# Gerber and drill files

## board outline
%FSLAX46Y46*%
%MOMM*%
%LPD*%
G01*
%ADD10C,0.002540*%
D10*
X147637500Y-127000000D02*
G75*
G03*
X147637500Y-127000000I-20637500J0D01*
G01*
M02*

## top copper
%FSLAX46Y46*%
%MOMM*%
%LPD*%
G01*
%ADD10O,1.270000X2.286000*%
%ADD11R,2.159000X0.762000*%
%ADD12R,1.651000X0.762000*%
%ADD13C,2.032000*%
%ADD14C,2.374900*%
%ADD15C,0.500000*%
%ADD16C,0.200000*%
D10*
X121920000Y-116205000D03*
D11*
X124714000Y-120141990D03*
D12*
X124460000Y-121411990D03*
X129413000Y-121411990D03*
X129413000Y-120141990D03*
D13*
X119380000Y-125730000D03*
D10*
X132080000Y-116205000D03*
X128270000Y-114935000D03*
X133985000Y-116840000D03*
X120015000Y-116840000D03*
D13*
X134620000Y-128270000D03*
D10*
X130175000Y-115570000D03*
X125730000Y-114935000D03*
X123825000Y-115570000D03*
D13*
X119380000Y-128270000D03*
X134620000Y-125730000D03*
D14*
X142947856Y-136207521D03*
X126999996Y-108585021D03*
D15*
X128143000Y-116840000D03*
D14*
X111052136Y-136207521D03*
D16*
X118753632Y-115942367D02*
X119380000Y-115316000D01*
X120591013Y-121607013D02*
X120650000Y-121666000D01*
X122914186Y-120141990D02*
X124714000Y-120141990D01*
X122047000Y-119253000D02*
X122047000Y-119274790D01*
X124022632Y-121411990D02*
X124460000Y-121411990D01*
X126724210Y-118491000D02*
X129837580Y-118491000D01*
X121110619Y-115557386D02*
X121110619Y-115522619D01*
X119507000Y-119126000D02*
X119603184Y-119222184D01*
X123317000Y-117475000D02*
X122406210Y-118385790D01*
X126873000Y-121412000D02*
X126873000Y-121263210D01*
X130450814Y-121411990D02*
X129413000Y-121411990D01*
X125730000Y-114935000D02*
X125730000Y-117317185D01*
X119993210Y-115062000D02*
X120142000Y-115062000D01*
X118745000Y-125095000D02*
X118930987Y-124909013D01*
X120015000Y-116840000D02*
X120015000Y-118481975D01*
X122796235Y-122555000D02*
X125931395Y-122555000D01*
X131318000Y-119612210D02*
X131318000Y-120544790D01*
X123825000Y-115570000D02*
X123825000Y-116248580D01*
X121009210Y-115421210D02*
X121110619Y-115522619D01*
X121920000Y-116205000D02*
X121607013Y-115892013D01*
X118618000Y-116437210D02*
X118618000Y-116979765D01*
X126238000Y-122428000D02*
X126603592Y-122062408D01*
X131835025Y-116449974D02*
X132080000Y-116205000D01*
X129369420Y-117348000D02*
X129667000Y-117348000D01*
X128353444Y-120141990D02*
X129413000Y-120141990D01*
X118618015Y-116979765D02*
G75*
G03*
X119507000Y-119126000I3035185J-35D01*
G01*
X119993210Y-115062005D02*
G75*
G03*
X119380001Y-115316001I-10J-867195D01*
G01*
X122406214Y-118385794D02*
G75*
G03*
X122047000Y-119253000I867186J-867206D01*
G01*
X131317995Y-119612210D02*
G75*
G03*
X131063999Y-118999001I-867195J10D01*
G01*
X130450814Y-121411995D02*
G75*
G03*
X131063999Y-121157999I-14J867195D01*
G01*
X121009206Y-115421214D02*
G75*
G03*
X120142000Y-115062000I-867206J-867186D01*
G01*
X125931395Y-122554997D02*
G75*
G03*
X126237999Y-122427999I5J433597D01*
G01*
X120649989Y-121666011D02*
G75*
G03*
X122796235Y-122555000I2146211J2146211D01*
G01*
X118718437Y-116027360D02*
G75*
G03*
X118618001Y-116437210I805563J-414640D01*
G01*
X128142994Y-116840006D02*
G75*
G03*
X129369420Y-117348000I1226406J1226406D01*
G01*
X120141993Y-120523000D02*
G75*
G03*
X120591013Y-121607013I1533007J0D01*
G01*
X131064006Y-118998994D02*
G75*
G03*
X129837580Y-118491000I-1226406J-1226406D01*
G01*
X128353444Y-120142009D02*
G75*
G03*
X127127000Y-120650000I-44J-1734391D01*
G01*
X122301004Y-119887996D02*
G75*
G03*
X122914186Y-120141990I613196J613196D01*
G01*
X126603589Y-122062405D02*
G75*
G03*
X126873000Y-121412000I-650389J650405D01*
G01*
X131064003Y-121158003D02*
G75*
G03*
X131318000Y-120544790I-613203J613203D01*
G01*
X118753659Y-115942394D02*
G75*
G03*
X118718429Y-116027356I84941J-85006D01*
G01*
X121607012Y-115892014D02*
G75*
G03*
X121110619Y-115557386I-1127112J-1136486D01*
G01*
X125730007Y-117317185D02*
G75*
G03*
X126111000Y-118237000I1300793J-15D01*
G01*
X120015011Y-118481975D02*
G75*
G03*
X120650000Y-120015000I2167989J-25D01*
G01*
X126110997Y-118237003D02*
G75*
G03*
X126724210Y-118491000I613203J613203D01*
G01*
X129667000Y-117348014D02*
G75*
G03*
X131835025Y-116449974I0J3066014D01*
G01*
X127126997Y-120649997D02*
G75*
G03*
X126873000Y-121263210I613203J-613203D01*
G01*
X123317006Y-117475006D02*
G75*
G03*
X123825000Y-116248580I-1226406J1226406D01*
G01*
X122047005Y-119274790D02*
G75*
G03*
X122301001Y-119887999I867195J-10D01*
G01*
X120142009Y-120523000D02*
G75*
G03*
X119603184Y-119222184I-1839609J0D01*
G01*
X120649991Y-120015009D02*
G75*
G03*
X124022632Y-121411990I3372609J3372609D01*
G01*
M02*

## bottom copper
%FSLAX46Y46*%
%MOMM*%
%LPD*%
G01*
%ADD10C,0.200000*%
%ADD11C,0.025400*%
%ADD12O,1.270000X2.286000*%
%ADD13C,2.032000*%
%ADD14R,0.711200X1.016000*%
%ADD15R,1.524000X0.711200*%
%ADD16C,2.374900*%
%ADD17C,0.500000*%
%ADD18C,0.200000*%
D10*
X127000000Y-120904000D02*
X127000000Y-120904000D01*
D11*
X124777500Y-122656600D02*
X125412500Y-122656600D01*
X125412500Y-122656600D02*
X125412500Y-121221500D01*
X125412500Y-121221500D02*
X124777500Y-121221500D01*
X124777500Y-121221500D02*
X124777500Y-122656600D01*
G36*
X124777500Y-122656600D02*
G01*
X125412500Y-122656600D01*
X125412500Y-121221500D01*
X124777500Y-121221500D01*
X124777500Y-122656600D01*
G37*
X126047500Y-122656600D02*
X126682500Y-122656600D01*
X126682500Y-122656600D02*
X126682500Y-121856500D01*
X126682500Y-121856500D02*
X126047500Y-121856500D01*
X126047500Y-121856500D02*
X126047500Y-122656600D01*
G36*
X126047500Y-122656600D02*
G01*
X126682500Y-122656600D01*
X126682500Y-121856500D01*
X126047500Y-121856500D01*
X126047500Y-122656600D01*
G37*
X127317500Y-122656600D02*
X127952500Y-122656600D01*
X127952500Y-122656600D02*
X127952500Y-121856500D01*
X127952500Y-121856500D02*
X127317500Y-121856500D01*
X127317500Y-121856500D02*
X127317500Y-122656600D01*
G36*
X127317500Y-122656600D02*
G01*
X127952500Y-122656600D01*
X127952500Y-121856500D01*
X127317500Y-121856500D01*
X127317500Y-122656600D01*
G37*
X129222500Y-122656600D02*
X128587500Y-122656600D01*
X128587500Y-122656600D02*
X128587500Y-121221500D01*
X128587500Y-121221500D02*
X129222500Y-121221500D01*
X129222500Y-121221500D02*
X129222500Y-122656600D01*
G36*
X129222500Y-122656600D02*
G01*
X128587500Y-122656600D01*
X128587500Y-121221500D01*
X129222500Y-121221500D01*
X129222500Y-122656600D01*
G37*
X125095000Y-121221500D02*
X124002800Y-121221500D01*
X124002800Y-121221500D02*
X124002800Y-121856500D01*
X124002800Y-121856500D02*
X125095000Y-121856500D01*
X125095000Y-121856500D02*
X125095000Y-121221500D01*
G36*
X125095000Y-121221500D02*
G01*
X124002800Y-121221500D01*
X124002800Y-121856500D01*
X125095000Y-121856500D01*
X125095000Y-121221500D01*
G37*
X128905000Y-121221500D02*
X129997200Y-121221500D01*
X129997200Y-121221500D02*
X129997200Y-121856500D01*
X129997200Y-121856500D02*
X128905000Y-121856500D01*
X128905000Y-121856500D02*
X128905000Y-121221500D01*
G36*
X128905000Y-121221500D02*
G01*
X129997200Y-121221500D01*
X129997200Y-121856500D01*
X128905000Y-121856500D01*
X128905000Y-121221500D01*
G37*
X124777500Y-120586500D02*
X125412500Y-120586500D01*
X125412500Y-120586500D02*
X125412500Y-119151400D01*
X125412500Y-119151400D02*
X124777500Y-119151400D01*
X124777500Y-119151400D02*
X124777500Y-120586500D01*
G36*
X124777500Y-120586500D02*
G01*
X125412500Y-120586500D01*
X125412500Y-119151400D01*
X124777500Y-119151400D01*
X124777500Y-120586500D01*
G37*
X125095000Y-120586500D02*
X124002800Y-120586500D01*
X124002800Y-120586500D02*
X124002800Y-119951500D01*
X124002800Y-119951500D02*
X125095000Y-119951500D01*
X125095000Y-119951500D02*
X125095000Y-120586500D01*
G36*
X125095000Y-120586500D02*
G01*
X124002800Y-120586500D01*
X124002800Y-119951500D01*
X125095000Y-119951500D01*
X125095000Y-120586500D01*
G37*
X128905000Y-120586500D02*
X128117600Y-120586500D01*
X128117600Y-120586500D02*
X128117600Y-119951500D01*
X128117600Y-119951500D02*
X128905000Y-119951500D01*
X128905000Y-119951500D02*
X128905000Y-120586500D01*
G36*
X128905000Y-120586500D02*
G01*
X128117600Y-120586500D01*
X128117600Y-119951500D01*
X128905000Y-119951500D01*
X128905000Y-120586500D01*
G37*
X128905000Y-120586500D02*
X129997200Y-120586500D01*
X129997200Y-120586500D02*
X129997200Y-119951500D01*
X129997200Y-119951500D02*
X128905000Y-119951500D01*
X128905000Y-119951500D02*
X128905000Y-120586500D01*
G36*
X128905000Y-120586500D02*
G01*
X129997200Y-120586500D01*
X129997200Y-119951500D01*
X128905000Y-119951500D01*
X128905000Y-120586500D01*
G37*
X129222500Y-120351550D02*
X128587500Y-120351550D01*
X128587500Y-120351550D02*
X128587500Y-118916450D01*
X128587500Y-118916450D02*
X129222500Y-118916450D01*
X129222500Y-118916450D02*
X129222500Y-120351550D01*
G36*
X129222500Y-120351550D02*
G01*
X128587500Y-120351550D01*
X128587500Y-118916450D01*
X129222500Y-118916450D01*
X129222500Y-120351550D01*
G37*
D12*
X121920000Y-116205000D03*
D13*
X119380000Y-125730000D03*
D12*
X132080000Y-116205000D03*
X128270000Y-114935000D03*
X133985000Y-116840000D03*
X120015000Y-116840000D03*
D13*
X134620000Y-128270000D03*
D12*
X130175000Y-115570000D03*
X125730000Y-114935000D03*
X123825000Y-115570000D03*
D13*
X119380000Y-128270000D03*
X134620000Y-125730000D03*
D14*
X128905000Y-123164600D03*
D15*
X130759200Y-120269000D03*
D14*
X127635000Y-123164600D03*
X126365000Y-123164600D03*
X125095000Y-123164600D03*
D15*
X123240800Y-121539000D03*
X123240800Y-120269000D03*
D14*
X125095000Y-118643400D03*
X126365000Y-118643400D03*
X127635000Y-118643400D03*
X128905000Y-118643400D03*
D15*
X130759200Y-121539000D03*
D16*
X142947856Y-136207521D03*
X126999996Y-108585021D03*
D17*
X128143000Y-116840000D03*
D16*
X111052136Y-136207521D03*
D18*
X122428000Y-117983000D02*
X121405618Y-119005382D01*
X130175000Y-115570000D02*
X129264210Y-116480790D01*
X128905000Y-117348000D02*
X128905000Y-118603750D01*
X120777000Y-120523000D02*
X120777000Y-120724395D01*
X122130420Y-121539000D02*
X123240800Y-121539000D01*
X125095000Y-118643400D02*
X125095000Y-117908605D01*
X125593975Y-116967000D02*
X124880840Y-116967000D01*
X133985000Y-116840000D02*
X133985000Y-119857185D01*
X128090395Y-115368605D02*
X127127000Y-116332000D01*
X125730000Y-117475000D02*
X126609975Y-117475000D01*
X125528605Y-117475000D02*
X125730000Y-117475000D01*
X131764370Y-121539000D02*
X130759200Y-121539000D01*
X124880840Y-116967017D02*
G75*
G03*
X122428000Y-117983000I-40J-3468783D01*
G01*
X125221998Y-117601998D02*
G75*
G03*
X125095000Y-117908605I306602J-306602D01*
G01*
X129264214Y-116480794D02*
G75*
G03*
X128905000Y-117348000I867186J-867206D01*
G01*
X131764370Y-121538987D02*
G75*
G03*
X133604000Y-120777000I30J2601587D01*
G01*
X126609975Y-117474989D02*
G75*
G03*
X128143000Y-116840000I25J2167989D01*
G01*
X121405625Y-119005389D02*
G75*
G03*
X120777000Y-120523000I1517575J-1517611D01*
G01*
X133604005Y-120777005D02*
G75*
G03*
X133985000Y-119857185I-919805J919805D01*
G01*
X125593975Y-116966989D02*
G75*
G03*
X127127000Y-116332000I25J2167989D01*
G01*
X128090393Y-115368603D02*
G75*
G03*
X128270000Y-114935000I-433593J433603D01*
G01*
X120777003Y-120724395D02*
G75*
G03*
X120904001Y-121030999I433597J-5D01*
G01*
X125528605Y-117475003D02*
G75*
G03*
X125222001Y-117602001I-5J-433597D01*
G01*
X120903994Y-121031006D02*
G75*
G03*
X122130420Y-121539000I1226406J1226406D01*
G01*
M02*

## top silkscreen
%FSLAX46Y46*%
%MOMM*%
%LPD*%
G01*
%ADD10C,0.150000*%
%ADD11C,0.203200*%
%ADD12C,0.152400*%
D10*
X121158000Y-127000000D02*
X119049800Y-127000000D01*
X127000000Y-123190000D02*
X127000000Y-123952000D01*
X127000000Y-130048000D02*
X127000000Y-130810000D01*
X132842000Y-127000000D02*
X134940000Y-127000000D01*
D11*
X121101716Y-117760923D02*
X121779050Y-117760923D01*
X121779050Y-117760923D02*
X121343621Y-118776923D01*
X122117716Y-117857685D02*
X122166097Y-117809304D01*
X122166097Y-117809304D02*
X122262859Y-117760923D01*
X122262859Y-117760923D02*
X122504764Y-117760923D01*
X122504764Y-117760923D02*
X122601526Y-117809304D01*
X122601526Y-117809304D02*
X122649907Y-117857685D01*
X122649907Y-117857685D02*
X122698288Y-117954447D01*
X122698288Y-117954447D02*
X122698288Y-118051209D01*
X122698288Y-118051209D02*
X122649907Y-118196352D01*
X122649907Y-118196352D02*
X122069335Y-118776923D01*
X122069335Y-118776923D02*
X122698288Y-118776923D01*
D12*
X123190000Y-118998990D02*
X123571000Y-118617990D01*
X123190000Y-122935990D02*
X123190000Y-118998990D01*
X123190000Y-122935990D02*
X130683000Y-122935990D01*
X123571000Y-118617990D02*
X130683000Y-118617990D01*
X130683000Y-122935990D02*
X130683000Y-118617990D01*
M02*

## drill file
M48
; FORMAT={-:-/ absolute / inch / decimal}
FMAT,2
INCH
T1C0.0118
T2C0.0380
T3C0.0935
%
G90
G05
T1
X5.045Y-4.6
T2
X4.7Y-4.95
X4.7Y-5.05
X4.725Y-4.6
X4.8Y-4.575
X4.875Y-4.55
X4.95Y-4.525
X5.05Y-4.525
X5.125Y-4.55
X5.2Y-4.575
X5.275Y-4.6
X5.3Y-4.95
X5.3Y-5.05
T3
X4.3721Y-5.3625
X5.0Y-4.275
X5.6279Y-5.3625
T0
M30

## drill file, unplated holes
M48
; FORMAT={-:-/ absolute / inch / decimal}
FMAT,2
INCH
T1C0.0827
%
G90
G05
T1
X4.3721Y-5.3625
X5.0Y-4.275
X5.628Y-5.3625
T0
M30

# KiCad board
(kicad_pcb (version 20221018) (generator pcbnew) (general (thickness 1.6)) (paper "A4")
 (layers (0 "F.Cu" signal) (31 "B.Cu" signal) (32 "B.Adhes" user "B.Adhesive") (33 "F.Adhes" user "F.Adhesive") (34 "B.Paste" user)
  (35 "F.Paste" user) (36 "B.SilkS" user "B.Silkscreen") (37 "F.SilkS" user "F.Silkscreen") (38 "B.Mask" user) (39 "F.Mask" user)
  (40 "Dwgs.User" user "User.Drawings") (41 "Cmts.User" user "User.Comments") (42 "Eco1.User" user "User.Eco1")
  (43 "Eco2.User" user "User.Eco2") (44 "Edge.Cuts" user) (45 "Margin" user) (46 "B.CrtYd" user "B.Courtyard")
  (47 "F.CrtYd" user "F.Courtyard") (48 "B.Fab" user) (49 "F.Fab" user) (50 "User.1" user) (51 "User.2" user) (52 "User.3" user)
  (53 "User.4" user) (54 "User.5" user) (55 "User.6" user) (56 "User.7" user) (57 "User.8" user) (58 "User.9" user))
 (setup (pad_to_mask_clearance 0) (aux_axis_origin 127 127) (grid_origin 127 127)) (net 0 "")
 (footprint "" (layer "F.Cu") (at 121.92 116.205)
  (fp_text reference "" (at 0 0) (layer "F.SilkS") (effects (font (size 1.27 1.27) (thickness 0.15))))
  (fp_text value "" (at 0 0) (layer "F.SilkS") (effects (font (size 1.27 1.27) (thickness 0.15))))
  (pad "1" thru_hole oval (at 0 0) (size 1.27 2.286) (drill 0.9652) (layers "*.Cu" "*.Mask") (thermal_bridge_angle 45)))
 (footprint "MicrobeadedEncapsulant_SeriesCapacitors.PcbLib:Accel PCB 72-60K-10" (layer "F.Cu") (at 127 120.904)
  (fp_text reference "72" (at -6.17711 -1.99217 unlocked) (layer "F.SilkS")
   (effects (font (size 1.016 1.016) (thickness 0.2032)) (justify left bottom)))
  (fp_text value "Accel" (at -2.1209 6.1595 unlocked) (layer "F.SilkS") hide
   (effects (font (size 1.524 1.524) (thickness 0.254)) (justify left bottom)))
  (fp_line (start -3.81 -1.90501) (end -3.429 -2.28601) (stroke (width 0.1524) (type solid)) (layer "F.SilkS"))
  (fp_line (start -3.81 2.03199) (end -3.81 -1.90501) (stroke (width 0.1524) (type solid)) (layer "F.SilkS"))
  (fp_line (start -3.81 2.03199) (end 3.683 2.03199) (stroke (width 0.1524) (type solid)) (layer "F.SilkS"))
  (fp_line (start -3.429 -2.28601) (end 3.683 -2.28601) (stroke (width 0.1524) (type solid)) (layer "F.SilkS"))
  (fp_line (start 3.683 2.03199) (end 3.683 -2.28601) (stroke (width 0.1524) (type solid)) (layer "F.SilkS"))
  (pad "1" smd rect (at -2.286 -0.76201 90) (size 0.762 2.159) (layers "F.Cu" "F.Paste" "F.Mask") (solder_mask_margin 0.1016)
   (thermal_bridge_angle 45))
  (pad "2" smd rect (at -2.54 0.50799 90) (size 0.762 1.651) (layers "F.Cu" "F.Paste" "F.Mask") (solder_mask_margin 0.1016)
   (thermal_bridge_angle 45))
  (pad "3" smd rect (at 2.413 0.50799 90) (size 0.762 1.651) (layers "F.Cu" "F.Paste" "F.Mask") (solder_mask_margin 0.1016)
   (thermal_bridge_angle 45))
  (pad "4" smd rect (at 2.413 -0.76201 90) (size 0.762 1.651) (layers "F.Cu" "F.Paste" "F.Mask") (solder_mask_margin 0.1016)
   (thermal_bridge_angle 45)))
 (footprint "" (layer "F.Cu") (at 119.38 125.73)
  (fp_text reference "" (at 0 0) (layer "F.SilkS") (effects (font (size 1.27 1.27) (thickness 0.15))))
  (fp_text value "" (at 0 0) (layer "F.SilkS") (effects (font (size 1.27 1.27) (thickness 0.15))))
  (pad "1" thru_hole circle (at 0 0) (size 2.032 2.032) (drill 0.9652) (layers "*.Cu" "*.Mask")))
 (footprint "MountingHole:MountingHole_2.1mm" (layer "F.Cu") (at 142.9512 136.2075)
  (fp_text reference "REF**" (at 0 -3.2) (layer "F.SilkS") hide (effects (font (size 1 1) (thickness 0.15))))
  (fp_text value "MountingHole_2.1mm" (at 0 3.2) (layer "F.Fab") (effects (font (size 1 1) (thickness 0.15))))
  (pad "" np_thru_hole circle (at 0 0) (size 2.1 2.1) (drill 2.1) (layers "*.Cu" "*.Mask")))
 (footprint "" (layer "F.Cu") (at 132.08 116.205)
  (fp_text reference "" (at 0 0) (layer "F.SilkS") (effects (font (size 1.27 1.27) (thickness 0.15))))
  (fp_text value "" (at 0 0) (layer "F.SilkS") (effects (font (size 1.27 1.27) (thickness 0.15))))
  (pad "1" thru_hole oval (at 0 0) (size 1.27 2.286) (drill 0.9652) (layers "*.Cu" "*.Mask") (thermal_bridge_angle 45)))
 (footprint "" (layer "F.Cu") (at 128.27 114.935)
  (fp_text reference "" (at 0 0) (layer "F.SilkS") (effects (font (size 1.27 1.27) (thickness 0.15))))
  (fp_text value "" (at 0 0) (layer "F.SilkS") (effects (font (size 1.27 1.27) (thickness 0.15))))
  (pad "1" thru_hole oval (at 0 0) (size 1.27 2.286) (drill 0.9652) (layers "*.Cu" "*.Mask") (thermal_bridge_angle 45)))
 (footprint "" (layer "F.Cu") (at 133.985 116.84)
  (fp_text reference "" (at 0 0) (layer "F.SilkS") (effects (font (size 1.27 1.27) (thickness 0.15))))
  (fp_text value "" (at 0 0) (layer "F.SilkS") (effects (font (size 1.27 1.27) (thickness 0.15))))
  (pad "1" thru_hole oval (at 0 0) (size 1.27 2.286) (drill 0.9652) (layers "*.Cu" "*.Mask") (thermal_bridge_angle 45)))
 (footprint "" (layer "F.Cu") (at 120.015 116.84)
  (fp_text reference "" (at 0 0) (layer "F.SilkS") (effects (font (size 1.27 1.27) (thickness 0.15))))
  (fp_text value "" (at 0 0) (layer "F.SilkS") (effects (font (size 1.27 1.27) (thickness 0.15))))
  (pad "1" thru_hole oval (at 0 0) (size 1.27 2.286) (drill 0.9652) (layers "*.Cu" "*.Mask") (thermal_bridge_angle 45)))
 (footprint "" (layer "F.Cu") (at 134.62 128.27)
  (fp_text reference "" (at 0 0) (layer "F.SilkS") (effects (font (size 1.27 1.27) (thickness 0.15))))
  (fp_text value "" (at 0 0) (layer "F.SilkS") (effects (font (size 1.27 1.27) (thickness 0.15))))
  (pad "1" thru_hole circle (at 0 0) (size 2.032 1.5) (drill 0.9652) (layers "*.Cu" "*.Mask")))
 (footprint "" (layer "F.Cu") (at 130.175 115.57)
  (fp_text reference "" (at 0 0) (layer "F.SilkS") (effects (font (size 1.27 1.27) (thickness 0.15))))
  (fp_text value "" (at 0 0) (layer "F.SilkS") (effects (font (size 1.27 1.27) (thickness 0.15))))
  (pad "1" thru_hole oval (at 0 0) (size 1.27 2.286) (drill 0.9652) (layers "*.Cu" "*.Mask") (thermal_bridge_angle 45)))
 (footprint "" (layer "F.Cu") (at 125.73 114.935)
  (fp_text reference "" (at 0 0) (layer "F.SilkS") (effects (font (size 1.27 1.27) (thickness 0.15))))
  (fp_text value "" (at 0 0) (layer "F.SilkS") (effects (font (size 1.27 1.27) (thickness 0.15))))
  (pad "1" thru_hole oval (at 0 0) (size 1.27 2.286) (drill 0.9652) (layers "*.Cu" "*.Mask") (thermal_bridge_angle 45)))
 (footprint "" (layer "F.Cu") (at 123.825 115.57)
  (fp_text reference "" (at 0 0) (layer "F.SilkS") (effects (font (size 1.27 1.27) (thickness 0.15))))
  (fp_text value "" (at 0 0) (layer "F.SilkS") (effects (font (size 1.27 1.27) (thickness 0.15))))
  (pad "1" thru_hole oval (at 0 0) (size 1.27 2.286) (drill 0.9652) (layers "*.Cu" "*.Mask") (thermal_bridge_angle 45)))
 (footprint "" (layer "F.Cu") (at 119.38 128.27)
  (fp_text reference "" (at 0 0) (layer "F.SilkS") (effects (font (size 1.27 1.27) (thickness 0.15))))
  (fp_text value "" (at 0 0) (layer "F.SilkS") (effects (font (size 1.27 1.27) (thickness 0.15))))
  (pad "1" thru_hole circle (at 0 0) (size 2.032 2.032) (drill 0.9652) (layers "*.Cu" "*.Mask")))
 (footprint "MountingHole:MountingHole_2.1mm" (layer "F.Cu") (at 127 108.585)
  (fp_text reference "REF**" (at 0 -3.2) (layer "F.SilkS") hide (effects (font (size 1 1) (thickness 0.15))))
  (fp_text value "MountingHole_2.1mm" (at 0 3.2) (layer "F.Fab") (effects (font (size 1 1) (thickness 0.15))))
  (pad "" np_thru_hole circle (at 0 0) (size 2.1 2.1) (drill 2.1) (layers "*.Cu" "*.Mask")))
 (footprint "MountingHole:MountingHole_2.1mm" (layer "F.Cu") (at 111.05134 136.2075)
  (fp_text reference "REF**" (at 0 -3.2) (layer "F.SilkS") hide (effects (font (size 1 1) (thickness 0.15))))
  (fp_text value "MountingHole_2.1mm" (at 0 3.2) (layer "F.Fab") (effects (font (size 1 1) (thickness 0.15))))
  (pad "" np_thru_hole circle (at 0 0) (size 2.1 2.1) (drill 2.1) (layers "*.Cu" "*.Mask")))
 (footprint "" (layer "F.Cu") (at 134.62 125.73)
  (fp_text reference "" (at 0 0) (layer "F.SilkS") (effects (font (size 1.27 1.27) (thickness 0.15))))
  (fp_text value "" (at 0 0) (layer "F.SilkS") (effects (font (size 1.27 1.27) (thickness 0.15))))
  (pad "1" thru_hole circle (at 0 0) (size 2.032 1.5) (drill 0.9652) (layers "*.Cu" "*.Mask")))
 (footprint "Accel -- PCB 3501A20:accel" (layer "B.Cu") (at 127 120.904 90)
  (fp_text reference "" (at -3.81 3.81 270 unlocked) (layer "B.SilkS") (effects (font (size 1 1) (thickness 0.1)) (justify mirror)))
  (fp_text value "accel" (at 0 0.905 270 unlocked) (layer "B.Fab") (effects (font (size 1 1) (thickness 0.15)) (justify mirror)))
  (fp_line (start 0 0) (end 0 0) (stroke (width 0.2) (type default)) (layer "B.Cu"))
  (fp_rect (start -1.7526 -2.2225) (end -0.3175 -1.5875) (stroke (width 0.0254) (type solid)) (fill solid) (layer "B.Cu"))
  (fp_rect (start -1.7526 -0.9525) (end -0.9525 -0.3175) (stroke (width 0.0254) (type solid)) (fill solid) (layer "B.Cu"))
  (fp_rect (start -1.7526 0.3175) (end -0.9525 0.9525) (stroke (width 0.0254) (type solid)) (fill solid) (layer "B.Cu"))
  (fp_rect (start -1.7526 2.2225) (end -0.3175 1.5875) (stroke (width 0.0254) (type solid)) (fill solid) (layer "B.Cu"))
  (fp_rect (start -0.3175 -1.905) (end -0.9525 -2.9972) (stroke (width 0.0254) (type solid)) (fill solid) (layer "B.Cu"))
  (fp_rect (start -0.3175 1.905) (end -0.9525 2.9972) (stroke (width 0.0254) (type solid)) (fill solid) (layer "B.Cu"))
  (fp_rect (start 0.3175 -2.2225) (end 1.7526 -1.5875) (stroke (width 0.0254) (type solid)) (fill solid) (layer "B.Cu"))
  (fp_rect (start 0.3175 -1.905) (end 0.9525 -2.9972) (stroke (width 0.0254) (type solid)) (fill solid) (layer "B.Cu"))
  (fp_rect (start 0.3175 1.905) (end 0.9525 1.1176) (stroke (width 0.0254) (type solid)) (fill solid) (layer "B.Cu"))
  (fp_rect (start 0.3175 1.905) (end 0.9525 2.9972) (stroke (width 0.0254) (type solid)) (fill solid) (layer "B.Cu"))
  (fp_rect (start 0.55245 2.2225) (end 1.98755 1.5875) (stroke (width 0.0254) (type solid)) (fill solid) (layer "B.Cu"))
  (pad "1" smd rect (at -2.2606 1.905) (size 0.7112 1.016) (layers "B.Cu" "B.Paste" "B.Mask") (thermal_bridge_angle 45))
  (pad "1" smd rect (at 0.635 3.7592 270) (size 0.7112 1.524) (layers "B.Cu" "B.Paste" "B.Mask") (thermal_bridge_angle 45))
  (pad "2" smd rect (at -2.2606 0.635) (size 0.7112 1.016) (layers "B.Cu" "B.Paste" "B.Mask") (thermal_bridge_angle 45))
  (pad "3" smd rect (at -2.2606 -0.635) (size 0.7112 1.016) (layers "B.Cu" "B.Paste" "B.Mask") (thermal_bridge_angle 45))
  (pad "4" smd rect (at -2.2606 -1.905) (size 0.7112 1.016) (layers "B.Cu" "B.Paste" "B.Mask") (thermal_bridge_angle 45))
  (pad "5" smd rect (at -0.635 -3.7592 270) (size 0.7112 1.524) (layers "B.Cu" "B.Paste" "B.Mask") (thermal_bridge_angle 45))
  (pad "6" smd rect (at 0.635 -3.7592 270) (size 0.7112 1.524) (layers "B.Cu" "B.Paste" "B.Mask") (thermal_bridge_angle 45))
  (pad "7" smd rect (at 2.2606 -1.905 180) (size 0.7112 1.016) (layers "B.Cu" "B.Paste" "B.Mask") (thermal_bridge_angle 45))
  (pad "8" smd rect (at 2.2606 -0.635 180) (size 0.7112 1.016) (layers "B.Cu" "B.Paste" "B.Mask") (thermal_bridge_angle 45))
  (pad "9" smd rect (at 2.2606 0.635 180) (size 0.7112 1.016) (layers "B.Cu" "B.Paste" "B.Mask") (thermal_bridge_angle 45))
  (pad "10" smd rect (at 2.2606 1.905 180) (size 0.7112 1.016) (layers "B.Cu" "B.Paste" "B.Mask") (thermal_bridge_angle 45))
  (pad "12" smd rect (at -0.635 3.7592 270) (size 0.7112 1.524) (layers "B.Cu" "B.Paste" "B.Mask") (thermal_bridge_angle 45)))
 (gr_line (start 121.158 127) (end 119.0498 127) (stroke (width 0.15) (type default)) (layer "F.SilkS"))
 (gr_line (start 127 123.19) (end 127 123.952) (stroke (width 0.15) (type default)) (layer "F.SilkS"))
 (gr_line (start 127 130.048) (end 127 130.81) (stroke (width 0.15) (type default)) (layer "F.SilkS"))
 (gr_line (start 132.842 127) (end 134.94 127) (stroke (width 0.15) (type default)) (layer "F.SilkS"))
 (gr_circle (center 127 127) (end 147.6375 127) (stroke (width 0.00254) (type default)) (fill none) (layer "Edge.Cuts"))
 (segment (start 118.753632 115.942367) (end 119.38 115.316) (width 0.2) (layer "F.Cu") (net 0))
 (segment (start 120.591013 121.607013) (end 120.65 121.666) (width 0.2) (layer "F.Cu") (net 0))
 (segment (start 122.914186 120.14199) (end 124.714 120.14199) (width 0.2) (layer "F.Cu") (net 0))
 (segment (start 122.047 119.253) (end 122.047 119.27479) (width 0.2) (layer "F.Cu") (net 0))
 (segment (start 124.022632 121.41199) (end 124.46 121.41199) (width 0.2) (layer "F.Cu") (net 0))
 (segment (start 126.72421 118.491) (end 129.83758 118.491) (width 0.2) (layer "F.Cu") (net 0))
 (segment (start 121.110619 115.557386) (end 121.110619 115.522619) (width 0.2) (layer "F.Cu") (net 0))
 (segment (start 119.507 119.126) (end 119.603184 119.222184) (width 0.2) (layer "F.Cu") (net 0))
 (segment (start 123.317 117.475) (end 122.40621 118.38579) (width 0.2) (layer "F.Cu") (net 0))
 (segment (start 126.873 121.412) (end 126.873 121.26321) (width 0.2) (layer "F.Cu") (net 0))
 (segment (start 130.450814 121.41199) (end 129.413 121.41199) (width 0.2) (layer "F.Cu") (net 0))
 (segment (start 125.73 114.935) (end 125.73 117.317185) (width 0.2) (layer "F.Cu") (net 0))
 (segment (start 119.99321 115.062) (end 120.142 115.062) (width 0.2) (layer "F.Cu") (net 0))
 (segment (start 118.745 125.095) (end 118.930987 124.909013) (width 0.2) (layer "F.Cu") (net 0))
 (segment (start 120.015 116.84) (end 120.015 118.481975) (width 0.2) (layer "F.Cu") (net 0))
 (segment (start 122.796235 122.555) (end 125.931395 122.555) (width 0.2) (layer "F.Cu") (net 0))
 (segment (start 131.318 119.61221) (end 131.318 120.54479) (width 0.2) (layer "F.Cu") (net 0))
 (segment (start 123.825 115.57) (end 123.825 116.24858) (width 0.2) (layer "F.Cu") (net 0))
 (segment (start 121.00921 115.42121) (end 121.110619 115.522619) (width 0.2) (layer "F.Cu") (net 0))
 (segment (start 121.92 116.205) (end 121.607013 115.892013) (width 0.2) (layer "F.Cu") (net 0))
 (segment (start 118.618 116.43721) (end 118.618 116.979765) (width 0.2) (layer "F.Cu") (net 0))
 (segment (start 126.238 122.428) (end 126.603592 122.062408) (width 0.2) (layer "F.Cu") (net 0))
 (segment (start 131.835025 116.449974) (end 132.08 116.205) (width 0.2) (layer "F.Cu") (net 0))
 (segment (start 129.36942 117.348) (end 129.667 117.348) (width 0.2) (layer "F.Cu") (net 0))
 (segment (start 128.353444 120.14199) (end 129.413 120.14199) (width 0.2) (layer "F.Cu") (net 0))
 (via (at 142.947856 136.207521) (size 2.3749) (drill 2.3749) (layers "F.Cu" "B.Cu") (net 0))
 (via (at 126.999996 108.585021) (size 2.3749) (drill 2.3749) (layers "F.Cu" "B.Cu") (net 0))
 (via (at 128.143 116.84) (size 0.5) (drill 0.3) (layers "F.Cu" "B.Cu") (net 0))
 (via (at 111.052136 136.207521) (size 2.3749) (drill 2.3749) (layers "F.Cu" "B.Cu") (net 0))
 (arc (start 118.618 116.979765) (mid 118.849044 118.141299) (end 119.507 119.126) (width 0.2) (layer "F.Cu") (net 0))
 (arc (start 119.38 115.316) (mid 119.661343 115.128013) (end 119.99321 115.062) (width 0.2) (layer "F.Cu") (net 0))
 (arc (start 122.40621 118.38579) (mid 122.140355 118.783669) (end 122.047 119.253) (width 0.2) (layer "F.Cu") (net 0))
 (arc (start 131.064 118.999) (mid 131.251987 119.280343) (end 131.318 119.61221) (width 0.2) (layer "F.Cu") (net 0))
 (arc (start 131.064 121.158) (mid 130.782668 121.34598) (end 130.450814 121.41199) (width 0.2) (layer "F.Cu") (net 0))
 (arc (start 120.142 115.062) (mid 120.611331 115.155356) (end 121.00921 115.42121) (width 0.2) (layer "F.Cu") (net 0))
 (arc (start 125.931395 122.555) (mid 126.097328 122.521994) (end 126.238 122.428) (width 0.2) (layer "F.Cu") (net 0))
 (arc (start 120.65 121.666) (mid 121.634701 122.323957) (end 122.796235 122.555) (width 0.2) (layer "F.Cu") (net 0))
 (arc (start 118.718429 116.027356) (mid 118.643987 116.226494) (end 118.618 116.43721) (width 0.2) (layer "F.Cu") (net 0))
 (arc (start 128.143 116.84) (mid 128.705686 117.215975) (end 129.36942 117.348) (width 0.2) (layer "F.Cu") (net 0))
 (arc (start 120.142 120.523) (mid 120.258695 121.109664) (end 120.591013 121.607013) (width 0.2) (layer "F.Cu") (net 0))
 (arc (start 129.83758 118.491) (mid 130.501313 118.623025) (end 131.064 118.999) (width 0.2) (layer "F.Cu") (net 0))
 (arc (start 127.127 120.65) (mid 127.689697 120.274018) (end 128.353444 120.14199) (width 0.2) (layer "F.Cu") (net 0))
 (arc (start 122.301 119.888) (mid 122.582332 120.075981) (end 122.914186 120.14199) (width 0.2) (layer "F.Cu") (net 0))
 (arc (start 126.603592 122.062408) (mid 126.802983 121.763999) (end 126.873 121.412) (width 0.2) (layer "F.Cu") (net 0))
 (arc (start 131.318 120.54479) (mid 131.251987 120.876656) (end 131.064 121.158) (width 0.2) (layer "F.Cu") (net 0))
 (arc (start 118.718429 116.027356) (mid 118.727578 115.981361) (end 118.753632 115.942367) (width 0.2) (layer "F.Cu") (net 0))
 (arc (start 121.607013 115.892013) (mid 121.374705 115.701358) (end 121.110619 115.557386) (width 0.2) (layer "F.Cu") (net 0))
 (arc (start 125.73 117.317185) (mid 125.829018 117.814985) (end 126.111 118.237) (width 0.2) (layer "F.Cu") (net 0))
 (arc (start 120.015 118.481975) (mid 120.180031 119.311642) (end 120.65 120.015) (width 0.2) (layer "F.Cu") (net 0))
 (arc (start 126.111 118.237) (mid 126.392343 118.424988) (end 126.72421 118.491) (width 0.2) (layer "F.Cu") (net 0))
 (arc (start 129.667 117.348) (mid 130.840327 117.114611) (end 131.835025 116.449974) (width 0.2) (layer "F.Cu") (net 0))
 (arc (start 126.873 121.26321) (mid 126.939013 120.931344) (end 127.127 120.65) (width 0.2) (layer "F.Cu") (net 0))
 (arc (start 123.825 116.24858) (mid 123.692975 116.912313) (end 123.317 117.475) (width 0.2) (layer "F.Cu") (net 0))
 (arc (start 122.047 119.27479) (mid 122.113012 119.606657) (end 122.301 119.888) (width 0.2) (layer "F.Cu") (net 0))
 (arc (start 119.603184 119.222184) (mid 120.001966 119.819003) (end 120.142 120.523) (width 0.2) (layer "F.Cu") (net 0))
 (arc (start 120.65 120.015) (mid 122.197376 121.048924) (end 124.022632 121.41199) (width 0.2) (layer "F.Cu") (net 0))
 (segment (start 122.428 117.983) (end 121.405618 119.005382) (width 0.2) (layer "B.Cu") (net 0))
 (segment (start 130.175 115.57) (end 129.26421 116.48079) (width 0.2) (layer "B.Cu") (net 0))
 (segment (start 128.905 117.348) (end 128.905 118.60375) (width 0.2) (layer "B.Cu") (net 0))
 (segment (start 120.777 120.523) (end 120.777 120.724395) (width 0.2) (layer "B.Cu") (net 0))
 (segment (start 122.13042 121.539) (end 123.2408 121.539) (width 0.2) (layer "B.Cu") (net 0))
 (segment (start 125.095 118.6434) (end 125.095 117.908605) (width 0.2) (layer "B.Cu") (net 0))
 (segment (start 125.593975 116.967) (end 124.88084 116.967) (width 0.2) (layer "B.Cu") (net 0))
 (segment (start 133.985 116.84) (end 133.985 119.857185) (width 0.2) (layer "B.Cu") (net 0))
 (segment (start 128.090395 115.368605) (end 127.127 116.332) (width 0.2) (layer "B.Cu") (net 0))
 (segment (start 125.73 117.475) (end 126.609975 117.475) (width 0.2) (layer "B.Cu") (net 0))
 (segment (start 125.528605 117.475) (end 125.73 117.475) (width 0.2) (layer "B.Cu") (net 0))
 (segment (start 131.76437 121.539) (end 130.7592 121.539) (width 0.2) (layer "B.Cu") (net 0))
 (arc (start 124.88084 116.967) (mid 123.553372 117.23105) (end 122.428 117.983) (width 0.2) (layer "B.Cu") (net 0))
 (arc (start 125.095 117.908605) (mid 125.128006 117.742672) (end 125.222 117.602) (width 0.2) (layer "B.Cu") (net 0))
 (arc (start 129.26421 116.48079) (mid 128.998355 116.878669) (end 128.905 117.348) (width 0.2) (layer "B.Cu") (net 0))
 (arc (start 133.604 120.777) (mid 132.759971 121.340962) (end 131.76437 121.539) (width 0.2) (layer "B.Cu") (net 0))
 (arc (start 126.609975 117.475) (mid 127.439642 117.309969) (end 128.143 116.84) (width 0.2) (layer "B.Cu") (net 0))
 (arc (start 121.405618 119.005382) (mid 120.940372 119.701671) (end 120.777 120.523) (width 0.2) (layer "B.Cu") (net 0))
 (arc (start 133.985 119.857185) (mid 133.885981 120.354985) (end 133.604 120.777) (width 0.2) (layer "B.Cu") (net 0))
 (arc (start 127.127 116.332) (mid 126.423643 116.801968) (end 125.593975 116.967) (width 0.2) (layer "B.Cu") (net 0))
 (arc (start 128.27 114.935) (mid 128.223322 115.169665) (end 128.090395 115.368605) (width 0.2) (layer "B.Cu") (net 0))
 (arc (start 120.777 120.724395) (mid 120.810006 120.890328) (end 120.904 121.031) (width 0.2) (layer "B.Cu") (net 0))
 (arc (start 125.222 117.602) (mid 125.362671 117.508006) (end 125.528605 117.475) (width 0.2) (layer "B.Cu") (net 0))
 (arc (start 120.904 121.031) (mid 121.466686 121.406975) (end 122.13042 121.539) (width 0.2) (layer "B.Cu") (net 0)))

